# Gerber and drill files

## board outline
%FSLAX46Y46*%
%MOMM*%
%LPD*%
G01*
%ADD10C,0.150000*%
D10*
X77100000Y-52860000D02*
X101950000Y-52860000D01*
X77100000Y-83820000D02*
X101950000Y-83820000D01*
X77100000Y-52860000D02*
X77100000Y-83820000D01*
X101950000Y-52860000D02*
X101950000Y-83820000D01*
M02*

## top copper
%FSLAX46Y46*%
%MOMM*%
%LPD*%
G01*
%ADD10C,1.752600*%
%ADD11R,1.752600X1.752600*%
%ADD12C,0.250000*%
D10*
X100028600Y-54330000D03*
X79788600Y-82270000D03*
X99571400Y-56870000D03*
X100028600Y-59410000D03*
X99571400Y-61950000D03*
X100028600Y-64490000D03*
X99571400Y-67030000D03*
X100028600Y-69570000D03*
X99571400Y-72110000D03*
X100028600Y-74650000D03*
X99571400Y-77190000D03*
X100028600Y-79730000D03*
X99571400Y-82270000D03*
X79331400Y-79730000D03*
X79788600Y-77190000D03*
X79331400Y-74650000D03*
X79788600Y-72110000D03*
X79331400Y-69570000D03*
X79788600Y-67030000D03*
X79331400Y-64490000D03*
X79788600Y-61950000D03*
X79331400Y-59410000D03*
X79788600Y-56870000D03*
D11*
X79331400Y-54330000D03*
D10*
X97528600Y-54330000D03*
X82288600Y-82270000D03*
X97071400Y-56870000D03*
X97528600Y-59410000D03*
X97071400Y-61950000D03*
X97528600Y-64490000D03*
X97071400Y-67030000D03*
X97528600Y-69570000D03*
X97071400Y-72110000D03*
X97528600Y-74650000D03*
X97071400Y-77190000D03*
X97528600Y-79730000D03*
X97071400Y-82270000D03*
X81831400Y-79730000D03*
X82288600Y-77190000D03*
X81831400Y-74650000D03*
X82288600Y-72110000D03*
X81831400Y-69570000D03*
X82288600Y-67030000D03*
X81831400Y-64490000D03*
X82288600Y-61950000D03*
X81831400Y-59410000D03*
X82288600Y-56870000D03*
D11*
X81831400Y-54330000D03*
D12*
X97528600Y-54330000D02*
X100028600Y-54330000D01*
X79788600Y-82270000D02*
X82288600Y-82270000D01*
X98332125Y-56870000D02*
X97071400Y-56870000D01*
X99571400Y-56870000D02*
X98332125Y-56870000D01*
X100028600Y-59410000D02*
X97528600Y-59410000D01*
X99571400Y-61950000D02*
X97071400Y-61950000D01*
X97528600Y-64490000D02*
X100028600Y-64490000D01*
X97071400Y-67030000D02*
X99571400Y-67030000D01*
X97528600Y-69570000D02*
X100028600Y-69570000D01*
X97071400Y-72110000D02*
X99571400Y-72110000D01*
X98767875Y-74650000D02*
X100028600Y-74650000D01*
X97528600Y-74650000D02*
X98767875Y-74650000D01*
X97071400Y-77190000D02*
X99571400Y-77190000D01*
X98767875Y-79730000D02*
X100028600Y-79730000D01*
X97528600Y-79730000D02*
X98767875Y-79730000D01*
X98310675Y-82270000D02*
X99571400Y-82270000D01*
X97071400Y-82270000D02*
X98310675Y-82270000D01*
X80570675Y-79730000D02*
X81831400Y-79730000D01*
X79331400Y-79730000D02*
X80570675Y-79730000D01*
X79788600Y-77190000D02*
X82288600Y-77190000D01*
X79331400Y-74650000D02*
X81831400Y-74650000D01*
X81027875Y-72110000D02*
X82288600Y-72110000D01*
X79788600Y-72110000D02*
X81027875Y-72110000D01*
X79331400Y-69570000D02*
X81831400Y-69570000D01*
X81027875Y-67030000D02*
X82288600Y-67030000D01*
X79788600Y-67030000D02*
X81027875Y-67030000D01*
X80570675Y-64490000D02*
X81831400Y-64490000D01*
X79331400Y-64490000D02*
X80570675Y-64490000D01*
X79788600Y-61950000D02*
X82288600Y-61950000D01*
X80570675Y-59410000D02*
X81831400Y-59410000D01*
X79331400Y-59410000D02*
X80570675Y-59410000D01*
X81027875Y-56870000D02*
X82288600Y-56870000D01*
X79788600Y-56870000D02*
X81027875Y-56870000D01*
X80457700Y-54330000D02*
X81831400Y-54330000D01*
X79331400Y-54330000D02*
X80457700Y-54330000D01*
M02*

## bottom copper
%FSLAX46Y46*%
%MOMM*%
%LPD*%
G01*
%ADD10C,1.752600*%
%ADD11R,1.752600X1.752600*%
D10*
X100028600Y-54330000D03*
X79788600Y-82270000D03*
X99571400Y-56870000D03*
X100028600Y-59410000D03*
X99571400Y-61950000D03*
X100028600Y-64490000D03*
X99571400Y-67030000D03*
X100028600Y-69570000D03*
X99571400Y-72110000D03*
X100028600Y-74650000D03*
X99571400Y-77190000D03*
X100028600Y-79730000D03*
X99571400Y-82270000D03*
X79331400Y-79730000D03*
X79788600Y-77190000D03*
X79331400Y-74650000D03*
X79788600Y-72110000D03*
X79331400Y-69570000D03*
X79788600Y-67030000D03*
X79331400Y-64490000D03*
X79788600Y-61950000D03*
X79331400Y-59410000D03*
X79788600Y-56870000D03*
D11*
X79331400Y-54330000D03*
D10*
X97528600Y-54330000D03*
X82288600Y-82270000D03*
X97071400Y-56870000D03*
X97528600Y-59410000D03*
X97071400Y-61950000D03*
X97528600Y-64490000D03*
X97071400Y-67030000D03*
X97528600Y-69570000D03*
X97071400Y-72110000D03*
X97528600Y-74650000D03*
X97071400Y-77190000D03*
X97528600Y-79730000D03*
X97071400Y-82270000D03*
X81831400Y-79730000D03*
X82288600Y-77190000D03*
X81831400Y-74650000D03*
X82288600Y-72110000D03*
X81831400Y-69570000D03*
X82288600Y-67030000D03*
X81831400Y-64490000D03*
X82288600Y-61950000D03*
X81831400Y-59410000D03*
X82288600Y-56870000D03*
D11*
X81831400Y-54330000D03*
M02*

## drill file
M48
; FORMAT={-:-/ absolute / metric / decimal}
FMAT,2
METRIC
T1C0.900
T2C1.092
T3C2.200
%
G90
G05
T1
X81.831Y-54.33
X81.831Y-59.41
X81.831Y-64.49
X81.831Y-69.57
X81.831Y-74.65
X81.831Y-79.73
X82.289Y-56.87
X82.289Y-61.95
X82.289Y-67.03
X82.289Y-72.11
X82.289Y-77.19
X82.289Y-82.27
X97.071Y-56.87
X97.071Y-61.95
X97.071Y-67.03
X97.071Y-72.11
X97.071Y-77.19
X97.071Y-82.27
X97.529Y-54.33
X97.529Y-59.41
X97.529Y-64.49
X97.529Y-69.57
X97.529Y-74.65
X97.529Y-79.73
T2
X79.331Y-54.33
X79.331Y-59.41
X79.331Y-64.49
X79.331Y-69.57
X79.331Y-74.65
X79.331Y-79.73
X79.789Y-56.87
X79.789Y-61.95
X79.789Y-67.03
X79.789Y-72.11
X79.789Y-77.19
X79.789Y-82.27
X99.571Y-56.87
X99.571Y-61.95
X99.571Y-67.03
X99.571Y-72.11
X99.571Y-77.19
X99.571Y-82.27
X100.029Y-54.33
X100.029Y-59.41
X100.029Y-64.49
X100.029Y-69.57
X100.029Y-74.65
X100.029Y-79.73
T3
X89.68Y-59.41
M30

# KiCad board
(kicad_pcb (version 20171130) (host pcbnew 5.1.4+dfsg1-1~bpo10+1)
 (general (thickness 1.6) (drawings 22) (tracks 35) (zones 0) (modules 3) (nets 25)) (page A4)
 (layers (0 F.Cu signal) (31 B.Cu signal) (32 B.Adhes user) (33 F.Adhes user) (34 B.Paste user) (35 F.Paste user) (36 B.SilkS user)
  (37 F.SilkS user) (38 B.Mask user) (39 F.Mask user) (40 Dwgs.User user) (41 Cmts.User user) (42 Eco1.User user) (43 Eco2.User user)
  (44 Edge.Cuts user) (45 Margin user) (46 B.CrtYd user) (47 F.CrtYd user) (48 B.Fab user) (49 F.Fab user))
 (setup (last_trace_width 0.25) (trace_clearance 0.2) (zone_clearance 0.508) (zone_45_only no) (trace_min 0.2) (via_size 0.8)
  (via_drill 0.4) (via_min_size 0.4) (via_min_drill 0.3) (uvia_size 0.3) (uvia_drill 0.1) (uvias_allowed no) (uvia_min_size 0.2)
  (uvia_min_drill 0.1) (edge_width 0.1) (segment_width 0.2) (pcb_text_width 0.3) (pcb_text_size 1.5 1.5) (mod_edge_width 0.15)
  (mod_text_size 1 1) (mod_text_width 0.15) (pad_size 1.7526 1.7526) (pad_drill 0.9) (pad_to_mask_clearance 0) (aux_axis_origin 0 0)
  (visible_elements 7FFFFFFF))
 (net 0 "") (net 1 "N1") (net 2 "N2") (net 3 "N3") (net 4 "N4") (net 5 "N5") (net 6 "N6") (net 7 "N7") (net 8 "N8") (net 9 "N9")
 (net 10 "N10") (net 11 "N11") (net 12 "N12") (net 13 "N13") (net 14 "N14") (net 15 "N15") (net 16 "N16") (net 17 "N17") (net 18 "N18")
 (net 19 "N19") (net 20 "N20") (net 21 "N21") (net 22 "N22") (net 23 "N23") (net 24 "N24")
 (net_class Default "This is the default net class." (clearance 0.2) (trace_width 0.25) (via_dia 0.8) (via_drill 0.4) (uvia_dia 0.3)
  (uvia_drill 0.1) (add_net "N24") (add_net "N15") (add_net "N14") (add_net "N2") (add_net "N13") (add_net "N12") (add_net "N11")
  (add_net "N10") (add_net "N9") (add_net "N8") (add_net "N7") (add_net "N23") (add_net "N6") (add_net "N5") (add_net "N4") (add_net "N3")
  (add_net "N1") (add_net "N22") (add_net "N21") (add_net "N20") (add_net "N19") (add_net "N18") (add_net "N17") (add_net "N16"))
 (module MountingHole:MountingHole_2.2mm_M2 (layer F.Cu) (at 89.68 59.41)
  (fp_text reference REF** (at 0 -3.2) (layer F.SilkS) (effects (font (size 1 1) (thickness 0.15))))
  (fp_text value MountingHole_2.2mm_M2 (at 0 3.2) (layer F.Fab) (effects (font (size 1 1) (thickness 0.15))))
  (pad 1 np_thru_hole circle (at 0 0) (size 2.2 2.2) (drill 2.2) (layers *.Cu *.Mask)))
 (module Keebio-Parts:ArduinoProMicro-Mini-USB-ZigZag (layer F.Cu) (at 89.68 68.3 270)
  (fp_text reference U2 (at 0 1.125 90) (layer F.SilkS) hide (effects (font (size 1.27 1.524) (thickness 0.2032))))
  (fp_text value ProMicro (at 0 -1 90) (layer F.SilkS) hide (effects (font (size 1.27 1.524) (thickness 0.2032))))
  (pad 24 thru_hole circle (at -13.97 -10.3486 270) (size 1.7526 1.7526) (drill 1.0922) (layers *.Cu *.SilkS *.Mask) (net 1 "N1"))
  (pad 12 thru_hole circle (at 13.97 9.8914 270) (size 1.7526 1.7526) (drill 1.0922) (layers *.Cu *.SilkS *.Mask) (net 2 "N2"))
  (pad 23 thru_hole circle (at -11.43 -9.8914 270) (size 1.7526 1.7526) (drill 1.0922) (layers *.Cu *.SilkS *.Mask) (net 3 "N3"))
  (pad 22 thru_hole circle (at -8.89 -10.3486 270) (size 1.7526 1.7526) (drill 1.0922) (layers *.Cu *.SilkS *.Mask) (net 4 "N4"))
  (pad 21 thru_hole circle (at -6.35 -9.8914 270) (size 1.7526 1.7526) (drill 1.0922) (layers *.Cu *.SilkS *.Mask) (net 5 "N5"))
  (pad 20 thru_hole circle (at -3.81 -10.3486 270) (size 1.7526 1.7526) (drill 1.0922) (layers *.Cu *.SilkS *.Mask) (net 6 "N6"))
  (pad 19 thru_hole circle (at -1.27 -9.8914 270) (size 1.7526 1.7526) (drill 1.0922) (layers *.Cu *.SilkS *.Mask) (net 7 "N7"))
  (pad 18 thru_hole circle (at 1.27 -10.3486 270) (size 1.7526 1.7526) (drill 1.0922) (layers *.Cu *.SilkS *.Mask) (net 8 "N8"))
  (pad 17 thru_hole circle (at 3.81 -9.8914 270) (size 1.7526 1.7526) (drill 1.0922) (layers *.Cu *.SilkS *.Mask) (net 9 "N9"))
  (pad 16 thru_hole circle (at 6.35 -10.3486 270) (size 1.7526 1.7526) (drill 1.0922) (layers *.Cu *.SilkS *.Mask) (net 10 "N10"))
  (pad 15 thru_hole circle (at 8.89 -9.8914 270) (size 1.7526 1.7526) (drill 1.0922) (layers *.Cu *.SilkS *.Mask) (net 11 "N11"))
  (pad 14 thru_hole circle (at 11.43 -10.3486 270) (size 1.7526 1.7526) (drill 1.0922) (layers *.Cu *.SilkS *.Mask) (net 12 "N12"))
  (pad 13 thru_hole circle (at 13.97 -9.8914 270) (size 1.7526 1.7526) (drill 1.0922) (layers *.Cu *.SilkS *.Mask) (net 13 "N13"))
  (pad 11 thru_hole circle (at 11.43 10.3486 270) (size 1.7526 1.7526) (drill 1.0922) (layers *.Cu *.SilkS *.Mask) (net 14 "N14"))
  (pad 10 thru_hole circle (at 8.89 9.8914 270) (size 1.7526 1.7526) (drill 1.0922) (layers *.Cu *.SilkS *.Mask) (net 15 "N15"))
  (pad 9 thru_hole circle (at 6.35 10.3486 270) (size 1.7526 1.7526) (drill 1.0922) (layers *.Cu *.SilkS *.Mask) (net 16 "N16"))
  (pad 8 thru_hole circle (at 3.81 9.8914 270) (size 1.7526 1.7526) (drill 1.0922) (layers *.Cu *.SilkS *.Mask) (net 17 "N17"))
  (pad 7 thru_hole circle (at 1.27 10.3486 270) (size 1.7526 1.7526) (drill 1.0922) (layers *.Cu *.SilkS *.Mask) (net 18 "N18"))
  (pad 6 thru_hole circle (at -1.27 9.8914 270) (size 1.7526 1.7526) (drill 1.0922) (layers *.Cu *.SilkS *.Mask) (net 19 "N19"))
  (pad 5 thru_hole circle (at -3.81 10.3486 270) (size 1.7526 1.7526) (drill 1.0922) (layers *.Cu *.SilkS *.Mask) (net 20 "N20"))
  (pad 4 thru_hole circle (at -6.35 9.8914 270) (size 1.7526 1.7526) (drill 1.0922) (layers *.Cu *.SilkS *.Mask) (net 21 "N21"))
  (pad 3 thru_hole circle (at -8.89 10.3486 270) (size 1.7526 1.7526) (drill 1.0922) (layers *.Cu *.SilkS *.Mask) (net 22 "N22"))
  (pad 2 thru_hole circle (at -11.43 9.8914 270) (size 1.7526 1.7526) (drill 1.0922) (layers *.Cu *.SilkS *.Mask) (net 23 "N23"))
  (pad 1 thru_hole rect (at -13.97 10.3486 270) (size 1.7526 1.7526) (drill 1.0922) (layers *.Cu *.SilkS *.Mask) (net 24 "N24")))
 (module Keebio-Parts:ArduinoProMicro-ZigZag (layer F.Cu) (at 89.68 68.3 270)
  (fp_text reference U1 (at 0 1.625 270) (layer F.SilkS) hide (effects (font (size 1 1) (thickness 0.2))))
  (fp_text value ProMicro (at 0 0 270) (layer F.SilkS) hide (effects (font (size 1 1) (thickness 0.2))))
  (pad 24 thru_hole circle (at -13.97 -7.8486 270) (size 1.7526 1.7526) (drill 0.9) (layers *.Cu *.SilkS *.Mask) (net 1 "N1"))
  (pad 12 thru_hole circle (at 13.97 7.3914 270) (size 1.7526 1.7526) (drill 0.9) (layers *.Cu *.SilkS *.Mask) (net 2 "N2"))
  (pad 23 thru_hole circle (at -11.43 -7.3914 270) (size 1.7526 1.7526) (drill 0.9) (layers *.Cu *.SilkS *.Mask) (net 3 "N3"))
  (pad 22 thru_hole circle (at -8.89 -7.8486 270) (size 1.7526 1.7526) (drill 0.9) (layers *.Cu *.SilkS *.Mask) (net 4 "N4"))
  (pad 21 thru_hole circle (at -6.35 -7.3914 270) (size 1.7526 1.7526) (drill 0.9) (layers *.Cu *.SilkS *.Mask) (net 5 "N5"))
  (pad 20 thru_hole circle (at -3.81 -7.8486 270) (size 1.7526 1.7526) (drill 0.9) (layers *.Cu *.SilkS *.Mask) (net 6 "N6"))
  (pad 19 thru_hole circle (at -1.27 -7.3914 270) (size 1.7526 1.7526) (drill 0.9) (layers *.Cu *.SilkS *.Mask) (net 7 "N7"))
  (pad 18 thru_hole circle (at 1.27 -7.8486 270) (size 1.7526 1.7526) (drill 0.9) (layers *.Cu *.SilkS *.Mask) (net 8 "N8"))
  (pad 17 thru_hole circle (at 3.81 -7.3914 270) (size 1.7526 1.7526) (drill 0.9) (layers *.Cu *.SilkS *.Mask) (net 9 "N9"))
  (pad 16 thru_hole circle (at 6.35 -7.8486 270) (size 1.7526 1.7526) (drill 0.9) (layers *.Cu *.SilkS *.Mask) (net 10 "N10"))
  (pad 15 thru_hole circle (at 8.89 -7.3914 270) (size 1.7526 1.7526) (drill 0.9) (layers *.Cu *.SilkS *.Mask) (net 11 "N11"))
  (pad 14 thru_hole circle (at 11.43 -7.8486 270) (size 1.7526 1.7526) (drill 0.9) (layers *.Cu *.SilkS *.Mask) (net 12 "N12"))
  (pad 13 thru_hole circle (at 13.97 -7.3914 270) (size 1.7526 1.7526) (drill 0.9) (layers *.Cu *.SilkS *.Mask) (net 13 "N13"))
  (pad 11 thru_hole circle (at 11.43 7.8486 270) (size 1.7526 1.7526) (drill 0.9) (layers *.Cu *.SilkS *.Mask) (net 14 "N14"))
  (pad 10 thru_hole circle (at 8.89 7.3914 270) (size 1.7526 1.7526) (drill 0.9) (layers *.Cu *.SilkS *.Mask) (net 15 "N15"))
  (pad 9 thru_hole circle (at 6.35 7.8486 270) (size 1.7526 1.7526) (drill 0.9) (layers *.Cu *.SilkS *.Mask) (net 16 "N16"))
  (pad 8 thru_hole circle (at 3.81 7.3914 270) (size 1.7526 1.7526) (drill 0.9) (layers *.Cu *.SilkS *.Mask) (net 17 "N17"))
  (pad 7 thru_hole circle (at 1.27 7.8486 270) (size 1.7526 1.7526) (drill 0.9) (layers *.Cu *.SilkS *.Mask) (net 18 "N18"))
  (pad 6 thru_hole circle (at -1.27 7.3914 270) (size 1.7526 1.7526) (drill 0.9) (layers *.Cu *.SilkS *.Mask) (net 19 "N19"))
  (pad 5 thru_hole circle (at -3.81 7.8486 270) (size 1.7526 1.7526) (drill 0.9) (layers *.Cu *.SilkS *.Mask) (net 20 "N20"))
  (pad 4 thru_hole circle (at -6.35 7.3914 270) (size 1.7526 1.7526) (drill 0.9) (layers *.Cu *.SilkS *.Mask) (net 21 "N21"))
  (pad 3 thru_hole circle (at -8.89 7.8486 270) (size 1.7526 1.7526) (drill 0.9) (layers *.Cu *.SilkS *.Mask) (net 22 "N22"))
  (pad 2 thru_hole circle (at -11.43 7.3914 270) (size 1.7526 1.7526) (drill 0.9) (layers *.Cu *.SilkS *.Mask) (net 23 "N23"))
  (pad 1 thru_hole rect (at -13.97 7.8486 270) (size 1.7526 1.7526) (drill 0.9) (layers *.Cu *.SilkS *.Mask) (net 24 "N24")))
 (gr_line (start 77.1 52.86) (end 101.95 52.86) (layer Edge.Cuts) (width 0.15))
 (gr_line (start 77.1 83.82) (end 101.95 83.82) (layer Edge.Cuts) (width 0.15))
 (gr_line (start 77.1 52.86) (end 77.1 83.82) (layer Edge.Cuts) (width 0.15))
 (gr_line (start 101.95 52.86) (end 101.95 83.82) (layer Edge.Cuts) (width 0.15))
 (segment (start 97.5286 54.33) (end 100.0286 54.33) (width 0.25) (layer F.Cu) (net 1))
 (segment (start 79.7886 82.27) (end 82.2886 82.27) (width 0.25) (layer F.Cu) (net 2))
 (segment (start 98.332125 56.87) (end 97.0714 56.87) (width 0.25) (layer F.Cu) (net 3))
 (segment (start 99.5714 56.87) (end 98.332125 56.87) (width 0.25) (layer F.Cu) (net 3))
 (segment (start 100.0286 59.41) (end 97.5286 59.41) (width 0.25) (layer F.Cu) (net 4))
 (segment (start 99.5714 61.95) (end 97.0714 61.95) (width 0.25) (layer F.Cu) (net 5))
 (segment (start 97.5286 64.49) (end 100.0286 64.49) (width 0.25) (layer F.Cu) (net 6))
 (segment (start 97.0714 67.03) (end 99.5714 67.03) (width 0.25) (layer F.Cu) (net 7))
 (segment (start 97.5286 69.57) (end 100.0286 69.57) (width 0.25) (layer F.Cu) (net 8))
 (segment (start 97.0714 72.11) (end 99.5714 72.11) (width 0.25) (layer F.Cu) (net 9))
 (segment (start 98.767875 74.65) (end 100.0286 74.65) (width 0.25) (layer F.Cu) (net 10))
 (segment (start 97.5286 74.65) (end 98.767875 74.65) (width 0.25) (layer F.Cu) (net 10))
 (segment (start 97.0714 77.19) (end 99.5714 77.19) (width 0.25) (layer F.Cu) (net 11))
 (segment (start 98.767875 79.73) (end 100.0286 79.73) (width 0.25) (layer F.Cu) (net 12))
 (segment (start 97.5286 79.73) (end 98.767875 79.73) (width 0.25) (layer F.Cu) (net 12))
 (segment (start 98.310675 82.27) (end 99.5714 82.27) (width 0.25) (layer F.Cu) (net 13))
 (segment (start 97.0714 82.27) (end 98.310675 82.27) (width 0.25) (layer F.Cu) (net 13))
 (segment (start 80.570675 79.73) (end 81.8314 79.73) (width 0.25) (layer F.Cu) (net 14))
 (segment (start 79.3314 79.73) (end 80.570675 79.73) (width 0.25) (layer F.Cu) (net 14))
 (segment (start 79.7886 77.19) (end 82.2886 77.19) (width 0.25) (layer F.Cu) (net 15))
 (segment (start 79.3314 74.65) (end 81.8314 74.65) (width 0.25) (layer F.Cu) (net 16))
 (segment (start 81.027875 72.11) (end 82.2886 72.11) (width 0.25) (layer F.Cu) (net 17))
 (segment (start 79.7886 72.11) (end 81.027875 72.11) (width 0.25) (layer F.Cu) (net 17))
 (segment (start 79.3314 69.57) (end 81.8314 69.57) (width 0.25) (layer F.Cu) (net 18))
 (segment (start 81.027875 67.03) (end 82.2886 67.03) (width 0.25) (layer F.Cu) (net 19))
 (segment (start 79.7886 67.03) (end 81.027875 67.03) (width 0.25) (layer F.Cu) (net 19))
 (segment (start 80.570675 64.49) (end 81.8314 64.49) (width 0.25) (layer F.Cu) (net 20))
 (segment (start 79.3314 64.49) (end 80.570675 64.49) (width 0.25) (layer F.Cu) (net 20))
 (segment (start 79.7886 61.95) (end 82.2886 61.95) (width 0.25) (layer F.Cu) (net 21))
 (segment (start 80.570675 59.41) (end 81.8314 59.41) (width 0.25) (layer F.Cu) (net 22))
 (segment (start 79.3314 59.41) (end 80.570675 59.41) (width 0.25) (layer F.Cu) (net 22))
 (segment (start 81.027875 56.87) (end 82.2886 56.87) (width 0.25) (layer F.Cu) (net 23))
 (segment (start 79.7886 56.87) (end 81.027875 56.87) (width 0.25) (layer F.Cu) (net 23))
 (segment (start 80.4577 54.33) (end 81.8314 54.33) (width 0.25) (layer F.Cu) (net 24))
 (segment (start 79.3314 54.33) (end 80.4577 54.33) (width 0.25) (layer F.Cu) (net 24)))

